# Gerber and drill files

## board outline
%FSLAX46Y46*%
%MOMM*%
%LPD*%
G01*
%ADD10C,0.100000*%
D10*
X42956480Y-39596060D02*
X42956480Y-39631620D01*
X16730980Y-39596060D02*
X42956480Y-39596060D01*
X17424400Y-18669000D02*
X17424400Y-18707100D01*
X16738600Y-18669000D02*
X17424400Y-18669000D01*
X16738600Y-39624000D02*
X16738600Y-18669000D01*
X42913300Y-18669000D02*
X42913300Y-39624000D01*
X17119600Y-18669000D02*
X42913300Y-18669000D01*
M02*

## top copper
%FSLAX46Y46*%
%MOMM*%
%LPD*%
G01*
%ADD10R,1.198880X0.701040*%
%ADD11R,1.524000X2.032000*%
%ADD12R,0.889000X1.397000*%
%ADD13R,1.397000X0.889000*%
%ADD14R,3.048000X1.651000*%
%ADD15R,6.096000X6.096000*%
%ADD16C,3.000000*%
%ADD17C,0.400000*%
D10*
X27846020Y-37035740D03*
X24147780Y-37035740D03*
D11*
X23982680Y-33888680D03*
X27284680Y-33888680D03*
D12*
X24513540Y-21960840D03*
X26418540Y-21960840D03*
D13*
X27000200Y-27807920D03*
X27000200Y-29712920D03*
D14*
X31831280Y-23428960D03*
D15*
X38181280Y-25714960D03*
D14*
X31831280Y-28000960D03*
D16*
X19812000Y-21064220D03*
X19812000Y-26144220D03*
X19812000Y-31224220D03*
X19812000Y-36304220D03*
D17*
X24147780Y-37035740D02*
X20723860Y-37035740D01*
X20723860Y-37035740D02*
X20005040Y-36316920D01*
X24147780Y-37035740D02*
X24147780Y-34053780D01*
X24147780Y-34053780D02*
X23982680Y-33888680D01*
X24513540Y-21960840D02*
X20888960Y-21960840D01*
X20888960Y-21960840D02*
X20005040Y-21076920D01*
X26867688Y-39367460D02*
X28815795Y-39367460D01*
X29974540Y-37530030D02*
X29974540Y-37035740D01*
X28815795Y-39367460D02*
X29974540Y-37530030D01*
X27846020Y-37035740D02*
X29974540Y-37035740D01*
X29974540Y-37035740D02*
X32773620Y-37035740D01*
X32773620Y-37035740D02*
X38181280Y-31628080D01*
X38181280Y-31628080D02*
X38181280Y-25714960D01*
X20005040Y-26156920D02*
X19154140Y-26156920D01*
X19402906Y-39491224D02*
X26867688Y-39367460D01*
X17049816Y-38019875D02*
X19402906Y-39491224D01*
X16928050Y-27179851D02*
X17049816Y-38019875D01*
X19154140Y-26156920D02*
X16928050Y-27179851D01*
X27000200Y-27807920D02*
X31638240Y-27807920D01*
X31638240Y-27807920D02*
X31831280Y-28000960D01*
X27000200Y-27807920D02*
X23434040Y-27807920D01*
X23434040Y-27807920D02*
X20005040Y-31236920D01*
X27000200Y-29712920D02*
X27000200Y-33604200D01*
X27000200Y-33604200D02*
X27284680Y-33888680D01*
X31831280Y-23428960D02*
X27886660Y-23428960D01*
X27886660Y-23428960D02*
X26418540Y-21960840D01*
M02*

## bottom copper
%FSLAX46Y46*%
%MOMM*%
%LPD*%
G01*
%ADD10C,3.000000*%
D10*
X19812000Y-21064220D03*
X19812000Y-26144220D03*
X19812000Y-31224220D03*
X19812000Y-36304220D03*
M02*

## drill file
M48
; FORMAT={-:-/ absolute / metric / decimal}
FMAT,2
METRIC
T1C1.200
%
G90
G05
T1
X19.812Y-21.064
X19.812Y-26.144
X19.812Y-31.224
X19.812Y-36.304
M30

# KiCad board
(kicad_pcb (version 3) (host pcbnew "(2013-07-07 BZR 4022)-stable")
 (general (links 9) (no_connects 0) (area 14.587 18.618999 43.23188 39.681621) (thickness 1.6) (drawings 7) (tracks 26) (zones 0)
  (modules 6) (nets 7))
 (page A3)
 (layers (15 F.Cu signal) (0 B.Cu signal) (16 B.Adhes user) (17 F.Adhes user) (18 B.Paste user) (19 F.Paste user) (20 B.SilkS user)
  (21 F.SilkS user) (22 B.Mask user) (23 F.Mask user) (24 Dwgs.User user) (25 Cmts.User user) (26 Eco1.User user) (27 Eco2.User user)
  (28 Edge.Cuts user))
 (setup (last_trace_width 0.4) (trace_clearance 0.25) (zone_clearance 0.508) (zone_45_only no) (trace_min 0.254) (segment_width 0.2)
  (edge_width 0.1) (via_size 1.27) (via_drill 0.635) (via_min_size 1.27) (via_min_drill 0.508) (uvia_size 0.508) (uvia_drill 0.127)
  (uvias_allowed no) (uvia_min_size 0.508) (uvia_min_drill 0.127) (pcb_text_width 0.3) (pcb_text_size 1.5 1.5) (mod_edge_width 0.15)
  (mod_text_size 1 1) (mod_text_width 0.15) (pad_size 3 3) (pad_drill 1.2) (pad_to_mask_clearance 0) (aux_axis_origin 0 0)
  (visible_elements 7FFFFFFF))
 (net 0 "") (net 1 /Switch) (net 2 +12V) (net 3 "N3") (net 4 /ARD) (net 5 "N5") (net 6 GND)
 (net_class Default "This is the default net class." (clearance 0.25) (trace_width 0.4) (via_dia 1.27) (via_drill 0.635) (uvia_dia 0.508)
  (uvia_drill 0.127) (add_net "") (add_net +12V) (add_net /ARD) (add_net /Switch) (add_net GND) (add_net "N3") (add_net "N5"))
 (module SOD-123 (layer F.Cu) (at 25.9969 37.03574 180)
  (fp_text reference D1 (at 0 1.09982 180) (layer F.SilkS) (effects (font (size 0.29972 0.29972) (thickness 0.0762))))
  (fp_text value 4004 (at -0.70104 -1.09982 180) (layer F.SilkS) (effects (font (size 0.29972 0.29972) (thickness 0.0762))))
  (pad 1 smd rect (at -1.84912 0 180) (size 1.19888 0.70104) (layers F.Cu F.Paste F.Mask) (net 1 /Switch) (clearance 0.14986))
  (pad 2 smd rect (at 1.84912 0 180) (size 1.19888 0.70104) (layers F.Cu F.Paste F.Mask) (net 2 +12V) (clearance 0.14986)))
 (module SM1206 (layer F.Cu) (at 25.63368 33.88868)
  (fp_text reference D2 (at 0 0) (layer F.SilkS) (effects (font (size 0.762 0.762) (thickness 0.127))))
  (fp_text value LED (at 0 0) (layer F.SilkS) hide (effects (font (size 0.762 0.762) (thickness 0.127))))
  (pad 1 smd rect (at -1.651 0) (size 1.524 2.032) (layers F.Cu F.Paste F.Mask) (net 2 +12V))
  (pad 2 smd rect (at 1.651 0) (size 1.524 2.032) (layers F.Cu F.Paste F.Mask) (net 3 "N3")))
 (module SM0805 (layer F.Cu) (at 25.46604 21.96084)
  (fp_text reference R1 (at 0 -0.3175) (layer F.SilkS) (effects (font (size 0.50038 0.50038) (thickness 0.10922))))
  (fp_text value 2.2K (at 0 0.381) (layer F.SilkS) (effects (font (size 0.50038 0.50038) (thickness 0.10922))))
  (pad 1 smd rect (at -0.9525 0) (size 0.889 1.397) (layers F.Cu F.Paste F.Mask) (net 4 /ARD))
  (pad 2 smd rect (at 0.9525 0) (size 0.889 1.397) (layers F.Cu F.Paste F.Mask) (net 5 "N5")))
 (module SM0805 (layer F.Cu) (at 27.0002 28.76042 270)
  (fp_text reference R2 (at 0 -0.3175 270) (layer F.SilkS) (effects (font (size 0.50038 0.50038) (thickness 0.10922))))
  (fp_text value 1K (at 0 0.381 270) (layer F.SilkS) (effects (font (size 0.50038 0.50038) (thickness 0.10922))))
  (pad 1 smd rect (at -0.9525 0 270) (size 0.889 1.397) (layers F.Cu F.Paste F.Mask) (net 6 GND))
  (pad 2 smd rect (at 0.9525 0 270) (size 0.889 1.397) (layers F.Cu F.Paste F.Mask) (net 3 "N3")))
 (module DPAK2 (layer F.Cu) (at 31.83128 25.71496 270)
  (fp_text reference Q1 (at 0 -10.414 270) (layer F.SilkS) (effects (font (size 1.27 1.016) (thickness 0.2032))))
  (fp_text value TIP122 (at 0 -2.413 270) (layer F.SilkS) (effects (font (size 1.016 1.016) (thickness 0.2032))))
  (pad 1 smd rect (at -2.286 0 270) (size 1.651 3.048) (layers F.Cu F.Paste F.Mask) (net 5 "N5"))
  (pad 2 smd rect (at 0 -6.35 270) (size 6.096 6.096) (layers F.Cu F.Paste F.Mask) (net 1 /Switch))
  (pad 3 smd rect (at 2.286 0 270) (size 1.651 3.048) (layers F.Cu F.Paste F.Mask) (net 6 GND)))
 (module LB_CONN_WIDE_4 (layer F.Cu) (at 19.812 26.14422 270)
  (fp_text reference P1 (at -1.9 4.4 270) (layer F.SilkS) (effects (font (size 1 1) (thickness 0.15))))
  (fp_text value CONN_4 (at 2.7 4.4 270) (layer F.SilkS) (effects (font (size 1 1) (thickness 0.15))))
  (pad 1 thru_hole circle (at -5.08 0 270) (size 3 3) (drill 1.2) (layers *.Cu *.Mask F.SilkS) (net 4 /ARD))
  (pad 2 thru_hole circle (at 0 0 270) (size 3 3) (drill 1.2) (layers *.Cu *.Mask F.SilkS) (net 1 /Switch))
  (pad 3 thru_hole circle (at 5.08 0 270) (size 3 3) (drill 1.2) (layers *.Cu *.Mask F.SilkS) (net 6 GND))
  (pad 4 thru_hole circle (at 10.16 0 270) (size 3 3) (drill 1.2) (layers *.Cu *.Mask F.SilkS) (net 2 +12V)))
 (gr_line (start 42.95648 39.59606) (end 42.95648 39.63162) (angle 90) (layer Edge.Cuts) (width 0.1))
 (gr_line (start 16.73098 39.59606) (end 42.95648 39.59606) (angle 90) (layer Edge.Cuts) (width 0.1))
 (gr_line (start 17.4244 18.669) (end 17.4244 18.7071) (angle 90) (layer Edge.Cuts) (width 0.1))
 (gr_line (start 16.7386 18.669) (end 17.4244 18.669) (angle 90) (layer Edge.Cuts) (width 0.1))
 (gr_line (start 16.7386 39.624) (end 16.7386 18.669) (angle 90) (layer Edge.Cuts) (width 0.1))
 (gr_line (start 42.9133 18.669) (end 42.9133 39.624) (angle 90) (layer Edge.Cuts) (width 0.1))
 (gr_line (start 17.1196 18.669) (end 42.9133 18.669) (angle 90) (layer Edge.Cuts) (width 0.1))
 (segment (start 24.14778 37.03574) (end 20.72386 37.03574) (width 0.4) (layer F.Cu) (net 2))
 (segment (start 20.72386 37.03574) (end 20.00504 36.31692) (width 0.4) (layer F.Cu) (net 2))
 (segment (start 24.14778 37.03574) (end 24.14778 34.05378) (width 0.4) (layer F.Cu) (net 2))
 (segment (start 24.14778 34.05378) (end 23.98268 33.88868) (width 0.4) (layer F.Cu) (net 2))
 (segment (start 24.51354 21.96084) (end 20.88896 21.96084) (width 0.4) (layer F.Cu) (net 4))
 (segment (start 20.88896 21.96084) (end 20.00504 21.07692) (width 0.4) (layer F.Cu) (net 4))
 (segment (start 26.867688 39.36746) (end 28.815795 39.36746) (width 0.4) (layer F.Cu) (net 1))
 (segment (start 29.97454 37.53003) (end 29.97454 37.03574) (width 0.4) (layer F.Cu) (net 1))
 (segment (start 28.815795 39.36746) (end 29.97454 37.53003) (width 0.4) (layer F.Cu) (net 1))
 (segment (start 27.84602 37.03574) (end 29.97454 37.03574) (width 0.4) (layer F.Cu) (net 1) (status 400000))
 (segment (start 29.97454 37.03574) (end 32.77362 37.03574) (width 0.4) (layer F.Cu) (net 1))
 (segment (start 32.77362 37.03574) (end 38.18128 31.62808) (width 0.4) (layer F.Cu) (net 1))
 (segment (start 38.18128 31.62808) (end 38.18128 25.71496) (width 0.4) (layer F.Cu) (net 1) (status 800000))
 (segment (start 20.00504 26.15692) (end 19.15414 26.15692) (width 0.4) (layer F.Cu) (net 1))
 (segment (start 19.402906 39.491224) (end 26.867688 39.36746) (width 0.4) (layer F.Cu) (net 1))
 (segment (start 17.049816 38.019875) (end 19.402906 39.491224) (width 0.4) (layer F.Cu) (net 1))
 (segment (start 16.92805 27.179851) (end 17.049816 38.019875) (width 0.4) (layer F.Cu) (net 1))
 (segment (start 19.15414 26.15692) (end 16.92805 27.179851) (width 0.4) (layer F.Cu) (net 1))
 (segment (start 27.0002 27.80792) (end 31.63824 27.80792) (width 0.4) (layer F.Cu) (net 6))
 (segment (start 31.63824 27.80792) (end 31.83128 28.00096) (width 0.4) (layer F.Cu) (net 6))
 (segment (start 27.0002 27.80792) (end 23.43404 27.80792) (width 0.4) (layer F.Cu) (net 6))
 (segment (start 23.43404 27.80792) (end 20.00504 31.23692) (width 0.4) (layer F.Cu) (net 6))
 (segment (start 27.0002 29.71292) (end 27.0002 33.6042) (width 0.4) (layer F.Cu) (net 3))
 (segment (start 27.0002 33.6042) (end 27.28468 33.88868) (width 0.4) (layer F.Cu) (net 3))
 (segment (start 31.83128 23.42896) (end 27.88666 23.42896) (width 0.4) (layer F.Cu) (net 5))
 (segment (start 27.88666 23.42896) (end 26.41854 21.96084) (width 0.4) (layer F.Cu) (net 5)))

